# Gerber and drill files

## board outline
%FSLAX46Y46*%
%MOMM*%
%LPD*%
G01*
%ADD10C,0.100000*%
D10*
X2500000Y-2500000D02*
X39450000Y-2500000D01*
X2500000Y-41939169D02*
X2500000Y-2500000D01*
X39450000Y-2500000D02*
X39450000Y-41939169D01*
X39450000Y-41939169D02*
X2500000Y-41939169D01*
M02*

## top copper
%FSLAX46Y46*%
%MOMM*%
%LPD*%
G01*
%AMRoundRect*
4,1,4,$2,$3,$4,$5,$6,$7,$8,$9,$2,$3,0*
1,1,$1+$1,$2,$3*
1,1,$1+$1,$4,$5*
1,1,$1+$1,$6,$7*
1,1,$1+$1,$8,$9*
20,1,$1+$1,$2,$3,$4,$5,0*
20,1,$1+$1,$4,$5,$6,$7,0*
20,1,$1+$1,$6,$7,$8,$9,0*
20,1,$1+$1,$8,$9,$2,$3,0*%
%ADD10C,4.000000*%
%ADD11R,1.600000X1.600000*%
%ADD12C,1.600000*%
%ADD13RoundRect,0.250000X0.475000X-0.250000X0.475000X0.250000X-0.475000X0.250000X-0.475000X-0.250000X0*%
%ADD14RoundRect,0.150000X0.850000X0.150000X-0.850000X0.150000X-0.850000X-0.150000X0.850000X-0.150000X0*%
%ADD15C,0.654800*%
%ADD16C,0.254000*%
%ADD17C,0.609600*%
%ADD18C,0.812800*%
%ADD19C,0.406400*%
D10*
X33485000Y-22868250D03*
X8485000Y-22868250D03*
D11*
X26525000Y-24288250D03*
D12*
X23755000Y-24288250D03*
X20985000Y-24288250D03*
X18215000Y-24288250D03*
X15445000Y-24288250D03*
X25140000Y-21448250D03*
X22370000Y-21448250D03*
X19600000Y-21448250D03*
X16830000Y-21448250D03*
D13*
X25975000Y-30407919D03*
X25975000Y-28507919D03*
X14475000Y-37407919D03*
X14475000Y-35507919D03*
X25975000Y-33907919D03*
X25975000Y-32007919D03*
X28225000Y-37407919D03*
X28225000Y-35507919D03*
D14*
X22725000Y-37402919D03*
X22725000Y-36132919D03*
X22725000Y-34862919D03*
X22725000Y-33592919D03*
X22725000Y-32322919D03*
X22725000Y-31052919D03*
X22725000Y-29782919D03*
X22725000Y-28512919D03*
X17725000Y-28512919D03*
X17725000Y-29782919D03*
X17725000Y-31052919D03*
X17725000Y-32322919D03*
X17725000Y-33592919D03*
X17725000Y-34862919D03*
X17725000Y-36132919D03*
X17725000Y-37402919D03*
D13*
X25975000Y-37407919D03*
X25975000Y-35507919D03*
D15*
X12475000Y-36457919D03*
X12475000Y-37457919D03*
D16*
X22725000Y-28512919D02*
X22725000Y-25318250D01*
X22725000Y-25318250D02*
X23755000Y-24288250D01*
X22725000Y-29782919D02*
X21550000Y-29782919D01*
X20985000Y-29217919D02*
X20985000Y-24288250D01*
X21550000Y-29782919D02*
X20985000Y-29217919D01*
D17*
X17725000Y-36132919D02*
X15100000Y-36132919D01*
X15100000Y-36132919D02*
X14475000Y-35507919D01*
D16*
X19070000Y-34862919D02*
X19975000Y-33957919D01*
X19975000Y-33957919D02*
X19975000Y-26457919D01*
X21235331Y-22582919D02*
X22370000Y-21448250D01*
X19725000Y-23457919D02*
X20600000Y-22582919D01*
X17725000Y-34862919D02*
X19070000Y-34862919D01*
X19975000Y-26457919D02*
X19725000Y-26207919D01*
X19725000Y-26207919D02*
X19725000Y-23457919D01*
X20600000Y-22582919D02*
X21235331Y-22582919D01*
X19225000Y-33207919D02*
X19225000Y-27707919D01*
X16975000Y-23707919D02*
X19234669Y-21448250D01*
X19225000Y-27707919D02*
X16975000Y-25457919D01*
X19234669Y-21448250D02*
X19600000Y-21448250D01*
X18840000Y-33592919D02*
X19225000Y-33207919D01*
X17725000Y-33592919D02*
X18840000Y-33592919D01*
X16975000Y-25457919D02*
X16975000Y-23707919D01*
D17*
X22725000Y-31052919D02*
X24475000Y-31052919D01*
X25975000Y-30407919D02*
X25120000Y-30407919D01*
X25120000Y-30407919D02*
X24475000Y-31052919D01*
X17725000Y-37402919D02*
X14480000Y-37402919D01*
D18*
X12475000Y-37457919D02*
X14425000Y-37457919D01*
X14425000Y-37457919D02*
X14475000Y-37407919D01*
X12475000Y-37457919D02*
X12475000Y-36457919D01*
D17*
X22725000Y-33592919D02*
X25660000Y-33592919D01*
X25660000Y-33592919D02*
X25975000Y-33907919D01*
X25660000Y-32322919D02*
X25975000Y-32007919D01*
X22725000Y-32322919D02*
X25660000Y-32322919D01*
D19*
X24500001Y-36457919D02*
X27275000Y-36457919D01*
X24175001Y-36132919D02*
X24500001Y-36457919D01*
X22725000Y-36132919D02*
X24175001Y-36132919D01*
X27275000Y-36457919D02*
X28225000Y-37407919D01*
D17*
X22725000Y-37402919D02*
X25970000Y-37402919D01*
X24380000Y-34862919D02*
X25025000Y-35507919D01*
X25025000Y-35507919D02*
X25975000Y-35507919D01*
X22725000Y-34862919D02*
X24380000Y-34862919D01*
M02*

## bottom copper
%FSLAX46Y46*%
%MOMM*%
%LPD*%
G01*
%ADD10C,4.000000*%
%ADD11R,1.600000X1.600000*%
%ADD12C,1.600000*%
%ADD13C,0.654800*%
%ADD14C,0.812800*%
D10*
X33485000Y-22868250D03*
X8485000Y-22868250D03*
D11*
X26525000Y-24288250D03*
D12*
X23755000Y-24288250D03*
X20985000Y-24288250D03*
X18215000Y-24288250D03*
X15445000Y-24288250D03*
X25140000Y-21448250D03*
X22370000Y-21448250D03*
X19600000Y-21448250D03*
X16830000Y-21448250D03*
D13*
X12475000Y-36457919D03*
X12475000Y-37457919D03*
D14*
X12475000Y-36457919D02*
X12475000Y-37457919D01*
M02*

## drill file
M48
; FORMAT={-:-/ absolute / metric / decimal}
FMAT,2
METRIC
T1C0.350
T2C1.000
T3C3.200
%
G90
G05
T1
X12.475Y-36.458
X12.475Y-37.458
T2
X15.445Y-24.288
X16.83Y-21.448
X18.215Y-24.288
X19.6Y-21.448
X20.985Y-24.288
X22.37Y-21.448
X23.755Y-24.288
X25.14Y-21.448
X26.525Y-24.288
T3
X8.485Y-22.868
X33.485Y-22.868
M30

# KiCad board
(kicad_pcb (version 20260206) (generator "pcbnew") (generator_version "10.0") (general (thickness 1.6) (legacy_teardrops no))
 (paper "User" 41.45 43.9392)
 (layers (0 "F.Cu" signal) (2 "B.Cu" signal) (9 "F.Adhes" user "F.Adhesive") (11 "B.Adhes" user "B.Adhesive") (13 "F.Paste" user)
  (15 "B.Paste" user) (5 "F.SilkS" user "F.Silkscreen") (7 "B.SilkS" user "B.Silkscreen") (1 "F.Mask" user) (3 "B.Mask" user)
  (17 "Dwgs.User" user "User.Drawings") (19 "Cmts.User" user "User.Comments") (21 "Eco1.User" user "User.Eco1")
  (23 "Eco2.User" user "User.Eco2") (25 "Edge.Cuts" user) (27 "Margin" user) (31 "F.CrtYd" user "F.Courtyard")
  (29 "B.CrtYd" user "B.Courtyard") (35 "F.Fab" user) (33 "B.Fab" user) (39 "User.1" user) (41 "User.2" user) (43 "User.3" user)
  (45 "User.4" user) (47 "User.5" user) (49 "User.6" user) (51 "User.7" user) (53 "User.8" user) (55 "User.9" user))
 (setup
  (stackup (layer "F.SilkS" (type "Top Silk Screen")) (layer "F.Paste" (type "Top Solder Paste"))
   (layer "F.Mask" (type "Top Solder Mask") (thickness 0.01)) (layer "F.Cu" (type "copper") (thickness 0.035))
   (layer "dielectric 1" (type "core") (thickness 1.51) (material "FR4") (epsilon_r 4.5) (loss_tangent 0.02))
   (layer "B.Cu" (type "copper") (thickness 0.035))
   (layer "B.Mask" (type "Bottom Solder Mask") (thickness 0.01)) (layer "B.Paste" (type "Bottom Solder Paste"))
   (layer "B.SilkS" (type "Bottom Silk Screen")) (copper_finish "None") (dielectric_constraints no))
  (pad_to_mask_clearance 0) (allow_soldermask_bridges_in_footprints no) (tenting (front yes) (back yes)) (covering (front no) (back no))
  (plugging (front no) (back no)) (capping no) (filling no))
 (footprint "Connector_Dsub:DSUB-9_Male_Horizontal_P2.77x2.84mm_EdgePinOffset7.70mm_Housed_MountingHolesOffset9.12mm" (layer "F.Cu")
  (at 26.525 24.28825 180)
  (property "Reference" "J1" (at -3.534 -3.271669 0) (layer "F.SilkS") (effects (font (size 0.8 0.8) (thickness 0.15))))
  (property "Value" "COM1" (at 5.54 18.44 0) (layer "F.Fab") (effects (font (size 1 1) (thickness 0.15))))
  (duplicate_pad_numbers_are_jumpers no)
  (pad "0" thru_hole circle (at -6.96 1.42 180) (size 4 4) (drill 3.2) (layers "*.Cu" "*.Mask") (remove_unused_layers no)
   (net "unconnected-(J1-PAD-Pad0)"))
  (pad "0" thru_hole circle (at 18.04 1.42 180) (size 4 4) (drill 3.2) (layers "*.Cu" "*.Mask") (remove_unused_layers no)
   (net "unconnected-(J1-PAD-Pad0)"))
  (pad "1" thru_hole rect (at 0 0 180) (size 1.6 1.6) (drill 1) (layers "*.Cu" "*.Mask") (remove_unused_layers no) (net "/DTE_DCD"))
  (pad "2" thru_hole circle (at 2.77 0 180) (size 1.6 1.6) (drill 1) (layers "*.Cu" "*.Mask") (remove_unused_layers no) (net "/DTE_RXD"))
  (pad "3" thru_hole circle (at 5.54 0 180) (size 1.6 1.6) (drill 1) (layers "*.Cu" "*.Mask") (remove_unused_layers no) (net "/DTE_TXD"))
  (pad "4" thru_hole circle (at 8.31 0 180) (size 1.6 1.6) (drill 1) (layers "*.Cu" "*.Mask") (remove_unused_layers no) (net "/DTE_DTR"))
  (pad "5" thru_hole circle (at 11.08 0 180) (size 1.6 1.6) (drill 1) (layers "*.Cu" "*.Mask") (remove_unused_layers no) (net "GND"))
  (pad "6" thru_hole circle (at 1.385 2.84 180) (size 1.6 1.6) (drill 1) (layers "*.Cu" "*.Mask") (remove_unused_layers no) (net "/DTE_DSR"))
  (pad "7" thru_hole circle (at 4.155 2.84 180) (size 1.6 1.6) (drill 1) (layers "*.Cu" "*.Mask") (remove_unused_layers no) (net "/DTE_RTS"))
  (pad "8" thru_hole circle (at 6.925 2.84 180) (size 1.6 1.6) (drill 1) (layers "*.Cu" "*.Mask") (remove_unused_layers no) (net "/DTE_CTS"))
  (pad "9" thru_hole circle (at 9.695 2.84 180) (size 1.6 1.6) (drill 1) (layers "*.Cu" "*.Mask") (remove_unused_layers no) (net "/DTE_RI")))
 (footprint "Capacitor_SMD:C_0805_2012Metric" (layer "F.Cu") (at 25.975 29.457919 90)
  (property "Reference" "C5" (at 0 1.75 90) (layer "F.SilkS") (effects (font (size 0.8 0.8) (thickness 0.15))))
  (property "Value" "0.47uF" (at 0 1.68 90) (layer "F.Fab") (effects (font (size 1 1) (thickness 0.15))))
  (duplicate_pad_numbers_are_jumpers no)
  (pad "1" smd roundrect (at -0.95 0 90) (size 1 1.45) (layers "F.Cu" "F.Mask" "F.Paste") (roundrect_rratio 0.25) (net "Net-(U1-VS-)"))
  (pad "2" smd roundrect (at 0.95 0 90) (size 1 1.45) (layers "F.Cu" "F.Mask" "F.Paste") (roundrect_rratio 0.25) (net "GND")))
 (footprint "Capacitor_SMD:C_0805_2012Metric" (layer "F.Cu") (at 14.475 36.457919 90)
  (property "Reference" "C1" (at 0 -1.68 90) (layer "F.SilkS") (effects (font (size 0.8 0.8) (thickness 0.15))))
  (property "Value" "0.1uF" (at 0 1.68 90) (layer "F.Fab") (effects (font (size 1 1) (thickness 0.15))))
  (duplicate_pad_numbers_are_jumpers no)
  (pad "1" smd roundrect (at -0.95 0 90) (size 1 1.45) (layers "F.Cu" "F.Mask" "F.Paste") (roundrect_rratio 0.25) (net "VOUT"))
  (pad "2" smd roundrect (at 0.95 0 90) (size 1 1.45) (layers "F.Cu" "F.Mask" "F.Paste") (roundrect_rratio 0.25) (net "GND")))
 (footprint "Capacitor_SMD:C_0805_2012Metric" (layer "F.Cu") (at 25.975 32.957919 90)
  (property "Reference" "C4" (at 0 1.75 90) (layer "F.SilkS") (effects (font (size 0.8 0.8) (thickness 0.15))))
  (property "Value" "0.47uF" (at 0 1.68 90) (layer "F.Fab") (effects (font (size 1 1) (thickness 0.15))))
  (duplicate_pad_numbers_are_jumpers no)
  (pad "1" smd roundrect (at -0.95 0 90) (size 1 1.45) (layers "F.Cu" "F.Mask" "F.Paste") (roundrect_rratio 0.25) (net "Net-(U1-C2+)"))
  (pad "2" smd roundrect (at 0.95 0 90) (size 1 1.45) (layers "F.Cu" "F.Mask" "F.Paste") (roundrect_rratio 0.25) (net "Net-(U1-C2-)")))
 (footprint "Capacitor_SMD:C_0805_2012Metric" (layer "F.Cu") (at 28.225 36.457919 90)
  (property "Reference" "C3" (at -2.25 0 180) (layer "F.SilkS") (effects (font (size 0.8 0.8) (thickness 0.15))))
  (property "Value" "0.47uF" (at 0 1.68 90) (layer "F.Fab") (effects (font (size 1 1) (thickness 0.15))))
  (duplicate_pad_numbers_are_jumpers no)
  (pad "1" smd roundrect (at -0.95 0 90) (size 1 1.45) (layers "F.Cu" "F.Mask" "F.Paste") (roundrect_rratio 0.25) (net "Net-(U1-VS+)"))
  (pad "2" smd roundrect (at 0.95 0 90) (size 1 1.45) (layers "F.Cu" "F.Mask" "F.Paste") (roundrect_rratio 0.25) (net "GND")))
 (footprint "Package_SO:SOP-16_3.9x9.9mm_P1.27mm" (layer "F.Cu") (at 20.225 32.957919 180)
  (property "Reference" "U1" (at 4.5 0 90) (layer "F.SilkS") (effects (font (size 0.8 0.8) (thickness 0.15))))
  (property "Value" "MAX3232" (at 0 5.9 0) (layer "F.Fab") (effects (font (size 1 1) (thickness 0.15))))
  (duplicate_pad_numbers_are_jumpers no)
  (pad "1" smd roundrect (at -2.5 -4.445 180) (size 2 0.6) (layers "F.Cu" "F.Mask" "F.Paste") (roundrect_rratio 0.25) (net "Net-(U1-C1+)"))
  (pad "2" smd roundrect (at -2.5 -3.175 180) (size 2 0.6) (layers "F.Cu" "F.Mask" "F.Paste") (roundrect_rratio 0.25) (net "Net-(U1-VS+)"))
  (pad "3" smd roundrect (at -2.5 -1.905 180) (size 2 0.6) (layers "F.Cu" "F.Mask" "F.Paste") (roundrect_rratio 0.25) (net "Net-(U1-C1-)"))
  (pad "4" smd roundrect (at -2.5 -0.635 180) (size 2 0.6) (layers "F.Cu" "F.Mask" "F.Paste") (roundrect_rratio 0.25) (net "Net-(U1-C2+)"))
  (pad "5" smd roundrect (at -2.5 0.635 180) (size 2 0.6) (layers "F.Cu" "F.Mask" "F.Paste") (roundrect_rratio 0.25) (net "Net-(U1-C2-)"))
  (pad "6" smd roundrect (at -2.5 1.905 180) (size 2 0.6) (layers "F.Cu" "F.Mask" "F.Paste") (roundrect_rratio 0.25) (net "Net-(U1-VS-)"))
  (pad "7" smd roundrect (at -2.5 3.175 180) (size 2 0.6) (layers "F.Cu" "F.Mask" "F.Paste") (roundrect_rratio 0.25) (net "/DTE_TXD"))
  (pad "8" smd roundrect (at -2.5 4.445 180) (size 2 0.6) (layers "F.Cu" "F.Mask" "F.Paste") (roundrect_rratio 0.25) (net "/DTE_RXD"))
  (pad "9" smd roundrect (at 2.5 4.445 180) (size 2 0.6) (layers "F.Cu" "F.Mask" "F.Paste") (roundrect_rratio 0.25) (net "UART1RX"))
  (pad "10" smd roundrect (at 2.5 3.175 180) (size 2 0.6) (layers "F.Cu" "F.Mask" "F.Paste") (roundrect_rratio 0.25) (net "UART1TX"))
  (pad "11" smd roundrect (at 2.5 1.905 180) (size 2 0.6) (layers "F.Cu" "F.Mask" "F.Paste") (roundrect_rratio 0.25) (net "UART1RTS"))
  (pad "12" smd roundrect (at 2.5 0.635 180) (size 2 0.6) (layers "F.Cu" "F.Mask" "F.Paste") (roundrect_rratio 0.25) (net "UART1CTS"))
  (pad "13" smd roundrect (at 2.5 -0.635 180) (size 2 0.6) (layers "F.Cu" "F.Mask" "F.Paste") (roundrect_rratio 0.25) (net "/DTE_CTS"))
  (pad "14" smd roundrect (at 2.5 -1.905 180) (size 2 0.6) (layers "F.Cu" "F.Mask" "F.Paste") (roundrect_rratio 0.25) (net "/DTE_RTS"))
  (pad "15" smd roundrect (at 2.5 -3.175 180) (size 2 0.6) (layers "F.Cu" "F.Mask" "F.Paste") (roundrect_rratio 0.25) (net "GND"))
  (pad "16" smd roundrect (at 2.5 -4.445 180) (size 2 0.6) (layers "F.Cu" "F.Mask" "F.Paste") (roundrect_rratio 0.25) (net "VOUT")))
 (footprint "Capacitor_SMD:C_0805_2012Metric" (layer "F.Cu") (at 25.975 36.457919 90)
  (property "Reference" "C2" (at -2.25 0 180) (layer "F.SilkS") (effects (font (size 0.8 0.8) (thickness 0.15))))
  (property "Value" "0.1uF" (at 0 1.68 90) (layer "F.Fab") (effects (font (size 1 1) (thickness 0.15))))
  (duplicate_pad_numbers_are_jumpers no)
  (pad "1" smd roundrect (at -0.95 0 90) (size 1 1.45) (layers "F.Cu" "F.Mask" "F.Paste") (roundrect_rratio 0.25) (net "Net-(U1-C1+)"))
  (pad "2" smd roundrect (at 0.95 0 90) (size 1 1.45) (layers "F.Cu" "F.Mask" "F.Paste") (roundrect_rratio 0.25) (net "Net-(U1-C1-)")))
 (gr_line (start 2.5 2.5) (end 39.45 2.5) (stroke (width 0.1) (type default)) (layer "Edge.Cuts"))
 (gr_line (start 2.5 41.939169) (end 2.5 2.5) (stroke (width 0.1) (type default)) (layer "Edge.Cuts"))
 (gr_line (start 39.45 2.5) (end 39.45 41.939169) (stroke (width 0.1) (type default)) (layer "Edge.Cuts"))
 (gr_line (start 39.45 41.939169) (end 2.5 41.939169) (stroke (width 0.1) (type default)) (layer "Edge.Cuts"))
 (segment (start 22.725 28.512919) (end 22.725 25.31825) (width 0.254) (layer "F.Cu") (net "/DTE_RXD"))
 (segment (start 22.725 25.31825) (end 23.755 24.28825) (width 0.254) (layer "F.Cu") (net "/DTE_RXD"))
 (segment (start 22.725 29.782919) (end 21.55 29.782919) (width 0.254) (layer "F.Cu") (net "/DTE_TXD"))
 (segment (start 20.985 29.217919) (end 20.985 24.28825) (width 0.254) (layer "F.Cu") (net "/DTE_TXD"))
 (segment (start 21.55 29.782919) (end 20.985 29.217919) (width 0.254) (layer "F.Cu") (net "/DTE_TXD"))
 (segment (start 17.725 36.132919) (end 15.1 36.132919) (width 0.6096) (layer "F.Cu") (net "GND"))
 (segment (start 15.1 36.132919) (end 14.475 35.507919) (width 0.6096) (layer "F.Cu") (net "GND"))
 (segment (start 19.07 34.862919) (end 19.975 33.957919) (width 0.254) (layer "F.Cu") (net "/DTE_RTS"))
 (segment (start 19.975 33.957919) (end 19.975 26.457919) (width 0.254) (layer "F.Cu") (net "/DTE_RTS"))
 (segment (start 21.235331 22.582919) (end 22.37 21.44825) (width 0.254) (layer "F.Cu") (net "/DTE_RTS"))
 (segment (start 19.725 23.457919) (end 20.6 22.582919) (width 0.254) (layer "F.Cu") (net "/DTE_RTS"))
 (segment (start 17.725 34.862919) (end 19.07 34.862919) (width 0.254) (layer "F.Cu") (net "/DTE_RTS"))
 (segment (start 19.975 26.457919) (end 19.725 26.207919) (width 0.254) (layer "F.Cu") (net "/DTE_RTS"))
 (segment (start 19.725 26.207919) (end 19.725 23.457919) (width 0.254) (layer "F.Cu") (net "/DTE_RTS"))
 (segment (start 20.6 22.582919) (end 21.235331 22.582919) (width 0.254) (layer "F.Cu") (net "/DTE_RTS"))
 (segment (start 19.225 33.207919) (end 19.225 27.707919) (width 0.254) (layer "F.Cu") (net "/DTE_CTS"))
 (segment (start 16.975 23.707919) (end 19.234669 21.44825) (width 0.254) (layer "F.Cu") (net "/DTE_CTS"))
 (segment (start 19.225 27.707919) (end 16.975 25.457919) (width 0.254) (layer "F.Cu") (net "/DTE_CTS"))
 (segment (start 19.234669 21.44825) (end 19.6 21.44825) (width 0.254) (layer "F.Cu") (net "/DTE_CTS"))
 (segment (start 18.84 33.592919) (end 19.225 33.207919) (width 0.254) (layer "F.Cu") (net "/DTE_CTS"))
 (segment (start 17.725 33.592919) (end 18.84 33.592919) (width 0.254) (layer "F.Cu") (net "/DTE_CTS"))
 (segment (start 16.975 25.457919) (end 16.975 23.707919) (width 0.254) (layer "F.Cu") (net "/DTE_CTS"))
 (segment (start 22.725 31.052919) (end 24.475 31.052919) (width 0.6096) (layer "F.Cu") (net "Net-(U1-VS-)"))
 (segment (start 25.975 30.407919) (end 25.12 30.407919) (width 0.6096) (layer "F.Cu") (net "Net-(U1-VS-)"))
 (segment (start 25.12 30.407919) (end 24.475 31.052919) (width 0.6096) (layer "F.Cu") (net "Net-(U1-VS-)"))
 (segment (start 17.725 37.402919) (end 14.48 37.402919) (width 0.6096) (layer "F.Cu") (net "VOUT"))
 (segment (start 12.475 37.457919) (end 14.425 37.457919) (width 0.8128) (layer "F.Cu") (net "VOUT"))
 (segment (start 14.425 37.457919) (end 14.475 37.407919) (width 0.8128) (layer "F.Cu") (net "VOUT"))
 (segment (start 12.475 37.457919) (end 12.475 36.457919) (width 0.8128) (layer "F.Cu") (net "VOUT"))
 (via (at 12.475 36.457919) (size 0.6548) (drill 0.35) (layers "F.Cu" "B.Cu") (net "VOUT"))
 (via (at 12.475 37.457919) (size 0.6548) (drill 0.35) (layers "F.Cu" "B.Cu") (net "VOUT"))
 (segment (start 12.475 36.457919) (end 12.475 37.457919) (width 0.8128) (layer "B.Cu") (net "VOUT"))
 (segment (start 22.725 33.592919) (end 25.66 33.592919) (width 0.6096) (layer "F.Cu") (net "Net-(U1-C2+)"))
 (segment (start 25.66 33.592919) (end 25.975 33.907919) (width 0.6096) (layer "F.Cu") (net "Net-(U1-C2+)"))
 (segment (start 25.66 32.322919) (end 25.975 32.007919) (width 0.6096) (layer "F.Cu") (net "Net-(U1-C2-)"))
 (segment (start 22.725 32.322919) (end 25.66 32.322919) (width 0.6096) (layer "F.Cu") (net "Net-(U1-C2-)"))
 (segment (start 24.500001 36.457919) (end 27.275 36.457919) (width 0.4064) (layer "F.Cu") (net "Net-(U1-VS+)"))
 (segment (start 24.175001 36.132919) (end 24.500001 36.457919) (width 0.4064) (layer "F.Cu") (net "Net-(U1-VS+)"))
 (segment (start 22.725 36.132919) (end 24.175001 36.132919) (width 0.4064) (layer "F.Cu") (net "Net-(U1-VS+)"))
 (segment (start 27.275 36.457919) (end 28.225 37.407919) (width 0.4064) (layer "F.Cu") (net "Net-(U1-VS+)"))
 (segment (start 22.725 37.402919) (end 25.97 37.402919) (width 0.6096) (layer "F.Cu") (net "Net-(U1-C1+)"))
 (segment (start 24.38 34.862919) (end 25.025 35.507919) (width 0.6096) (layer "F.Cu") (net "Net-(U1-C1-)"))
 (segment (start 25.025 35.507919) (end 25.975 35.507919) (width 0.6096) (layer "F.Cu") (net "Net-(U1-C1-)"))
 (segment (start 22.725 34.862919) (end 24.38 34.862919) (width 0.6096) (layer "F.Cu") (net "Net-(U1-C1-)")))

